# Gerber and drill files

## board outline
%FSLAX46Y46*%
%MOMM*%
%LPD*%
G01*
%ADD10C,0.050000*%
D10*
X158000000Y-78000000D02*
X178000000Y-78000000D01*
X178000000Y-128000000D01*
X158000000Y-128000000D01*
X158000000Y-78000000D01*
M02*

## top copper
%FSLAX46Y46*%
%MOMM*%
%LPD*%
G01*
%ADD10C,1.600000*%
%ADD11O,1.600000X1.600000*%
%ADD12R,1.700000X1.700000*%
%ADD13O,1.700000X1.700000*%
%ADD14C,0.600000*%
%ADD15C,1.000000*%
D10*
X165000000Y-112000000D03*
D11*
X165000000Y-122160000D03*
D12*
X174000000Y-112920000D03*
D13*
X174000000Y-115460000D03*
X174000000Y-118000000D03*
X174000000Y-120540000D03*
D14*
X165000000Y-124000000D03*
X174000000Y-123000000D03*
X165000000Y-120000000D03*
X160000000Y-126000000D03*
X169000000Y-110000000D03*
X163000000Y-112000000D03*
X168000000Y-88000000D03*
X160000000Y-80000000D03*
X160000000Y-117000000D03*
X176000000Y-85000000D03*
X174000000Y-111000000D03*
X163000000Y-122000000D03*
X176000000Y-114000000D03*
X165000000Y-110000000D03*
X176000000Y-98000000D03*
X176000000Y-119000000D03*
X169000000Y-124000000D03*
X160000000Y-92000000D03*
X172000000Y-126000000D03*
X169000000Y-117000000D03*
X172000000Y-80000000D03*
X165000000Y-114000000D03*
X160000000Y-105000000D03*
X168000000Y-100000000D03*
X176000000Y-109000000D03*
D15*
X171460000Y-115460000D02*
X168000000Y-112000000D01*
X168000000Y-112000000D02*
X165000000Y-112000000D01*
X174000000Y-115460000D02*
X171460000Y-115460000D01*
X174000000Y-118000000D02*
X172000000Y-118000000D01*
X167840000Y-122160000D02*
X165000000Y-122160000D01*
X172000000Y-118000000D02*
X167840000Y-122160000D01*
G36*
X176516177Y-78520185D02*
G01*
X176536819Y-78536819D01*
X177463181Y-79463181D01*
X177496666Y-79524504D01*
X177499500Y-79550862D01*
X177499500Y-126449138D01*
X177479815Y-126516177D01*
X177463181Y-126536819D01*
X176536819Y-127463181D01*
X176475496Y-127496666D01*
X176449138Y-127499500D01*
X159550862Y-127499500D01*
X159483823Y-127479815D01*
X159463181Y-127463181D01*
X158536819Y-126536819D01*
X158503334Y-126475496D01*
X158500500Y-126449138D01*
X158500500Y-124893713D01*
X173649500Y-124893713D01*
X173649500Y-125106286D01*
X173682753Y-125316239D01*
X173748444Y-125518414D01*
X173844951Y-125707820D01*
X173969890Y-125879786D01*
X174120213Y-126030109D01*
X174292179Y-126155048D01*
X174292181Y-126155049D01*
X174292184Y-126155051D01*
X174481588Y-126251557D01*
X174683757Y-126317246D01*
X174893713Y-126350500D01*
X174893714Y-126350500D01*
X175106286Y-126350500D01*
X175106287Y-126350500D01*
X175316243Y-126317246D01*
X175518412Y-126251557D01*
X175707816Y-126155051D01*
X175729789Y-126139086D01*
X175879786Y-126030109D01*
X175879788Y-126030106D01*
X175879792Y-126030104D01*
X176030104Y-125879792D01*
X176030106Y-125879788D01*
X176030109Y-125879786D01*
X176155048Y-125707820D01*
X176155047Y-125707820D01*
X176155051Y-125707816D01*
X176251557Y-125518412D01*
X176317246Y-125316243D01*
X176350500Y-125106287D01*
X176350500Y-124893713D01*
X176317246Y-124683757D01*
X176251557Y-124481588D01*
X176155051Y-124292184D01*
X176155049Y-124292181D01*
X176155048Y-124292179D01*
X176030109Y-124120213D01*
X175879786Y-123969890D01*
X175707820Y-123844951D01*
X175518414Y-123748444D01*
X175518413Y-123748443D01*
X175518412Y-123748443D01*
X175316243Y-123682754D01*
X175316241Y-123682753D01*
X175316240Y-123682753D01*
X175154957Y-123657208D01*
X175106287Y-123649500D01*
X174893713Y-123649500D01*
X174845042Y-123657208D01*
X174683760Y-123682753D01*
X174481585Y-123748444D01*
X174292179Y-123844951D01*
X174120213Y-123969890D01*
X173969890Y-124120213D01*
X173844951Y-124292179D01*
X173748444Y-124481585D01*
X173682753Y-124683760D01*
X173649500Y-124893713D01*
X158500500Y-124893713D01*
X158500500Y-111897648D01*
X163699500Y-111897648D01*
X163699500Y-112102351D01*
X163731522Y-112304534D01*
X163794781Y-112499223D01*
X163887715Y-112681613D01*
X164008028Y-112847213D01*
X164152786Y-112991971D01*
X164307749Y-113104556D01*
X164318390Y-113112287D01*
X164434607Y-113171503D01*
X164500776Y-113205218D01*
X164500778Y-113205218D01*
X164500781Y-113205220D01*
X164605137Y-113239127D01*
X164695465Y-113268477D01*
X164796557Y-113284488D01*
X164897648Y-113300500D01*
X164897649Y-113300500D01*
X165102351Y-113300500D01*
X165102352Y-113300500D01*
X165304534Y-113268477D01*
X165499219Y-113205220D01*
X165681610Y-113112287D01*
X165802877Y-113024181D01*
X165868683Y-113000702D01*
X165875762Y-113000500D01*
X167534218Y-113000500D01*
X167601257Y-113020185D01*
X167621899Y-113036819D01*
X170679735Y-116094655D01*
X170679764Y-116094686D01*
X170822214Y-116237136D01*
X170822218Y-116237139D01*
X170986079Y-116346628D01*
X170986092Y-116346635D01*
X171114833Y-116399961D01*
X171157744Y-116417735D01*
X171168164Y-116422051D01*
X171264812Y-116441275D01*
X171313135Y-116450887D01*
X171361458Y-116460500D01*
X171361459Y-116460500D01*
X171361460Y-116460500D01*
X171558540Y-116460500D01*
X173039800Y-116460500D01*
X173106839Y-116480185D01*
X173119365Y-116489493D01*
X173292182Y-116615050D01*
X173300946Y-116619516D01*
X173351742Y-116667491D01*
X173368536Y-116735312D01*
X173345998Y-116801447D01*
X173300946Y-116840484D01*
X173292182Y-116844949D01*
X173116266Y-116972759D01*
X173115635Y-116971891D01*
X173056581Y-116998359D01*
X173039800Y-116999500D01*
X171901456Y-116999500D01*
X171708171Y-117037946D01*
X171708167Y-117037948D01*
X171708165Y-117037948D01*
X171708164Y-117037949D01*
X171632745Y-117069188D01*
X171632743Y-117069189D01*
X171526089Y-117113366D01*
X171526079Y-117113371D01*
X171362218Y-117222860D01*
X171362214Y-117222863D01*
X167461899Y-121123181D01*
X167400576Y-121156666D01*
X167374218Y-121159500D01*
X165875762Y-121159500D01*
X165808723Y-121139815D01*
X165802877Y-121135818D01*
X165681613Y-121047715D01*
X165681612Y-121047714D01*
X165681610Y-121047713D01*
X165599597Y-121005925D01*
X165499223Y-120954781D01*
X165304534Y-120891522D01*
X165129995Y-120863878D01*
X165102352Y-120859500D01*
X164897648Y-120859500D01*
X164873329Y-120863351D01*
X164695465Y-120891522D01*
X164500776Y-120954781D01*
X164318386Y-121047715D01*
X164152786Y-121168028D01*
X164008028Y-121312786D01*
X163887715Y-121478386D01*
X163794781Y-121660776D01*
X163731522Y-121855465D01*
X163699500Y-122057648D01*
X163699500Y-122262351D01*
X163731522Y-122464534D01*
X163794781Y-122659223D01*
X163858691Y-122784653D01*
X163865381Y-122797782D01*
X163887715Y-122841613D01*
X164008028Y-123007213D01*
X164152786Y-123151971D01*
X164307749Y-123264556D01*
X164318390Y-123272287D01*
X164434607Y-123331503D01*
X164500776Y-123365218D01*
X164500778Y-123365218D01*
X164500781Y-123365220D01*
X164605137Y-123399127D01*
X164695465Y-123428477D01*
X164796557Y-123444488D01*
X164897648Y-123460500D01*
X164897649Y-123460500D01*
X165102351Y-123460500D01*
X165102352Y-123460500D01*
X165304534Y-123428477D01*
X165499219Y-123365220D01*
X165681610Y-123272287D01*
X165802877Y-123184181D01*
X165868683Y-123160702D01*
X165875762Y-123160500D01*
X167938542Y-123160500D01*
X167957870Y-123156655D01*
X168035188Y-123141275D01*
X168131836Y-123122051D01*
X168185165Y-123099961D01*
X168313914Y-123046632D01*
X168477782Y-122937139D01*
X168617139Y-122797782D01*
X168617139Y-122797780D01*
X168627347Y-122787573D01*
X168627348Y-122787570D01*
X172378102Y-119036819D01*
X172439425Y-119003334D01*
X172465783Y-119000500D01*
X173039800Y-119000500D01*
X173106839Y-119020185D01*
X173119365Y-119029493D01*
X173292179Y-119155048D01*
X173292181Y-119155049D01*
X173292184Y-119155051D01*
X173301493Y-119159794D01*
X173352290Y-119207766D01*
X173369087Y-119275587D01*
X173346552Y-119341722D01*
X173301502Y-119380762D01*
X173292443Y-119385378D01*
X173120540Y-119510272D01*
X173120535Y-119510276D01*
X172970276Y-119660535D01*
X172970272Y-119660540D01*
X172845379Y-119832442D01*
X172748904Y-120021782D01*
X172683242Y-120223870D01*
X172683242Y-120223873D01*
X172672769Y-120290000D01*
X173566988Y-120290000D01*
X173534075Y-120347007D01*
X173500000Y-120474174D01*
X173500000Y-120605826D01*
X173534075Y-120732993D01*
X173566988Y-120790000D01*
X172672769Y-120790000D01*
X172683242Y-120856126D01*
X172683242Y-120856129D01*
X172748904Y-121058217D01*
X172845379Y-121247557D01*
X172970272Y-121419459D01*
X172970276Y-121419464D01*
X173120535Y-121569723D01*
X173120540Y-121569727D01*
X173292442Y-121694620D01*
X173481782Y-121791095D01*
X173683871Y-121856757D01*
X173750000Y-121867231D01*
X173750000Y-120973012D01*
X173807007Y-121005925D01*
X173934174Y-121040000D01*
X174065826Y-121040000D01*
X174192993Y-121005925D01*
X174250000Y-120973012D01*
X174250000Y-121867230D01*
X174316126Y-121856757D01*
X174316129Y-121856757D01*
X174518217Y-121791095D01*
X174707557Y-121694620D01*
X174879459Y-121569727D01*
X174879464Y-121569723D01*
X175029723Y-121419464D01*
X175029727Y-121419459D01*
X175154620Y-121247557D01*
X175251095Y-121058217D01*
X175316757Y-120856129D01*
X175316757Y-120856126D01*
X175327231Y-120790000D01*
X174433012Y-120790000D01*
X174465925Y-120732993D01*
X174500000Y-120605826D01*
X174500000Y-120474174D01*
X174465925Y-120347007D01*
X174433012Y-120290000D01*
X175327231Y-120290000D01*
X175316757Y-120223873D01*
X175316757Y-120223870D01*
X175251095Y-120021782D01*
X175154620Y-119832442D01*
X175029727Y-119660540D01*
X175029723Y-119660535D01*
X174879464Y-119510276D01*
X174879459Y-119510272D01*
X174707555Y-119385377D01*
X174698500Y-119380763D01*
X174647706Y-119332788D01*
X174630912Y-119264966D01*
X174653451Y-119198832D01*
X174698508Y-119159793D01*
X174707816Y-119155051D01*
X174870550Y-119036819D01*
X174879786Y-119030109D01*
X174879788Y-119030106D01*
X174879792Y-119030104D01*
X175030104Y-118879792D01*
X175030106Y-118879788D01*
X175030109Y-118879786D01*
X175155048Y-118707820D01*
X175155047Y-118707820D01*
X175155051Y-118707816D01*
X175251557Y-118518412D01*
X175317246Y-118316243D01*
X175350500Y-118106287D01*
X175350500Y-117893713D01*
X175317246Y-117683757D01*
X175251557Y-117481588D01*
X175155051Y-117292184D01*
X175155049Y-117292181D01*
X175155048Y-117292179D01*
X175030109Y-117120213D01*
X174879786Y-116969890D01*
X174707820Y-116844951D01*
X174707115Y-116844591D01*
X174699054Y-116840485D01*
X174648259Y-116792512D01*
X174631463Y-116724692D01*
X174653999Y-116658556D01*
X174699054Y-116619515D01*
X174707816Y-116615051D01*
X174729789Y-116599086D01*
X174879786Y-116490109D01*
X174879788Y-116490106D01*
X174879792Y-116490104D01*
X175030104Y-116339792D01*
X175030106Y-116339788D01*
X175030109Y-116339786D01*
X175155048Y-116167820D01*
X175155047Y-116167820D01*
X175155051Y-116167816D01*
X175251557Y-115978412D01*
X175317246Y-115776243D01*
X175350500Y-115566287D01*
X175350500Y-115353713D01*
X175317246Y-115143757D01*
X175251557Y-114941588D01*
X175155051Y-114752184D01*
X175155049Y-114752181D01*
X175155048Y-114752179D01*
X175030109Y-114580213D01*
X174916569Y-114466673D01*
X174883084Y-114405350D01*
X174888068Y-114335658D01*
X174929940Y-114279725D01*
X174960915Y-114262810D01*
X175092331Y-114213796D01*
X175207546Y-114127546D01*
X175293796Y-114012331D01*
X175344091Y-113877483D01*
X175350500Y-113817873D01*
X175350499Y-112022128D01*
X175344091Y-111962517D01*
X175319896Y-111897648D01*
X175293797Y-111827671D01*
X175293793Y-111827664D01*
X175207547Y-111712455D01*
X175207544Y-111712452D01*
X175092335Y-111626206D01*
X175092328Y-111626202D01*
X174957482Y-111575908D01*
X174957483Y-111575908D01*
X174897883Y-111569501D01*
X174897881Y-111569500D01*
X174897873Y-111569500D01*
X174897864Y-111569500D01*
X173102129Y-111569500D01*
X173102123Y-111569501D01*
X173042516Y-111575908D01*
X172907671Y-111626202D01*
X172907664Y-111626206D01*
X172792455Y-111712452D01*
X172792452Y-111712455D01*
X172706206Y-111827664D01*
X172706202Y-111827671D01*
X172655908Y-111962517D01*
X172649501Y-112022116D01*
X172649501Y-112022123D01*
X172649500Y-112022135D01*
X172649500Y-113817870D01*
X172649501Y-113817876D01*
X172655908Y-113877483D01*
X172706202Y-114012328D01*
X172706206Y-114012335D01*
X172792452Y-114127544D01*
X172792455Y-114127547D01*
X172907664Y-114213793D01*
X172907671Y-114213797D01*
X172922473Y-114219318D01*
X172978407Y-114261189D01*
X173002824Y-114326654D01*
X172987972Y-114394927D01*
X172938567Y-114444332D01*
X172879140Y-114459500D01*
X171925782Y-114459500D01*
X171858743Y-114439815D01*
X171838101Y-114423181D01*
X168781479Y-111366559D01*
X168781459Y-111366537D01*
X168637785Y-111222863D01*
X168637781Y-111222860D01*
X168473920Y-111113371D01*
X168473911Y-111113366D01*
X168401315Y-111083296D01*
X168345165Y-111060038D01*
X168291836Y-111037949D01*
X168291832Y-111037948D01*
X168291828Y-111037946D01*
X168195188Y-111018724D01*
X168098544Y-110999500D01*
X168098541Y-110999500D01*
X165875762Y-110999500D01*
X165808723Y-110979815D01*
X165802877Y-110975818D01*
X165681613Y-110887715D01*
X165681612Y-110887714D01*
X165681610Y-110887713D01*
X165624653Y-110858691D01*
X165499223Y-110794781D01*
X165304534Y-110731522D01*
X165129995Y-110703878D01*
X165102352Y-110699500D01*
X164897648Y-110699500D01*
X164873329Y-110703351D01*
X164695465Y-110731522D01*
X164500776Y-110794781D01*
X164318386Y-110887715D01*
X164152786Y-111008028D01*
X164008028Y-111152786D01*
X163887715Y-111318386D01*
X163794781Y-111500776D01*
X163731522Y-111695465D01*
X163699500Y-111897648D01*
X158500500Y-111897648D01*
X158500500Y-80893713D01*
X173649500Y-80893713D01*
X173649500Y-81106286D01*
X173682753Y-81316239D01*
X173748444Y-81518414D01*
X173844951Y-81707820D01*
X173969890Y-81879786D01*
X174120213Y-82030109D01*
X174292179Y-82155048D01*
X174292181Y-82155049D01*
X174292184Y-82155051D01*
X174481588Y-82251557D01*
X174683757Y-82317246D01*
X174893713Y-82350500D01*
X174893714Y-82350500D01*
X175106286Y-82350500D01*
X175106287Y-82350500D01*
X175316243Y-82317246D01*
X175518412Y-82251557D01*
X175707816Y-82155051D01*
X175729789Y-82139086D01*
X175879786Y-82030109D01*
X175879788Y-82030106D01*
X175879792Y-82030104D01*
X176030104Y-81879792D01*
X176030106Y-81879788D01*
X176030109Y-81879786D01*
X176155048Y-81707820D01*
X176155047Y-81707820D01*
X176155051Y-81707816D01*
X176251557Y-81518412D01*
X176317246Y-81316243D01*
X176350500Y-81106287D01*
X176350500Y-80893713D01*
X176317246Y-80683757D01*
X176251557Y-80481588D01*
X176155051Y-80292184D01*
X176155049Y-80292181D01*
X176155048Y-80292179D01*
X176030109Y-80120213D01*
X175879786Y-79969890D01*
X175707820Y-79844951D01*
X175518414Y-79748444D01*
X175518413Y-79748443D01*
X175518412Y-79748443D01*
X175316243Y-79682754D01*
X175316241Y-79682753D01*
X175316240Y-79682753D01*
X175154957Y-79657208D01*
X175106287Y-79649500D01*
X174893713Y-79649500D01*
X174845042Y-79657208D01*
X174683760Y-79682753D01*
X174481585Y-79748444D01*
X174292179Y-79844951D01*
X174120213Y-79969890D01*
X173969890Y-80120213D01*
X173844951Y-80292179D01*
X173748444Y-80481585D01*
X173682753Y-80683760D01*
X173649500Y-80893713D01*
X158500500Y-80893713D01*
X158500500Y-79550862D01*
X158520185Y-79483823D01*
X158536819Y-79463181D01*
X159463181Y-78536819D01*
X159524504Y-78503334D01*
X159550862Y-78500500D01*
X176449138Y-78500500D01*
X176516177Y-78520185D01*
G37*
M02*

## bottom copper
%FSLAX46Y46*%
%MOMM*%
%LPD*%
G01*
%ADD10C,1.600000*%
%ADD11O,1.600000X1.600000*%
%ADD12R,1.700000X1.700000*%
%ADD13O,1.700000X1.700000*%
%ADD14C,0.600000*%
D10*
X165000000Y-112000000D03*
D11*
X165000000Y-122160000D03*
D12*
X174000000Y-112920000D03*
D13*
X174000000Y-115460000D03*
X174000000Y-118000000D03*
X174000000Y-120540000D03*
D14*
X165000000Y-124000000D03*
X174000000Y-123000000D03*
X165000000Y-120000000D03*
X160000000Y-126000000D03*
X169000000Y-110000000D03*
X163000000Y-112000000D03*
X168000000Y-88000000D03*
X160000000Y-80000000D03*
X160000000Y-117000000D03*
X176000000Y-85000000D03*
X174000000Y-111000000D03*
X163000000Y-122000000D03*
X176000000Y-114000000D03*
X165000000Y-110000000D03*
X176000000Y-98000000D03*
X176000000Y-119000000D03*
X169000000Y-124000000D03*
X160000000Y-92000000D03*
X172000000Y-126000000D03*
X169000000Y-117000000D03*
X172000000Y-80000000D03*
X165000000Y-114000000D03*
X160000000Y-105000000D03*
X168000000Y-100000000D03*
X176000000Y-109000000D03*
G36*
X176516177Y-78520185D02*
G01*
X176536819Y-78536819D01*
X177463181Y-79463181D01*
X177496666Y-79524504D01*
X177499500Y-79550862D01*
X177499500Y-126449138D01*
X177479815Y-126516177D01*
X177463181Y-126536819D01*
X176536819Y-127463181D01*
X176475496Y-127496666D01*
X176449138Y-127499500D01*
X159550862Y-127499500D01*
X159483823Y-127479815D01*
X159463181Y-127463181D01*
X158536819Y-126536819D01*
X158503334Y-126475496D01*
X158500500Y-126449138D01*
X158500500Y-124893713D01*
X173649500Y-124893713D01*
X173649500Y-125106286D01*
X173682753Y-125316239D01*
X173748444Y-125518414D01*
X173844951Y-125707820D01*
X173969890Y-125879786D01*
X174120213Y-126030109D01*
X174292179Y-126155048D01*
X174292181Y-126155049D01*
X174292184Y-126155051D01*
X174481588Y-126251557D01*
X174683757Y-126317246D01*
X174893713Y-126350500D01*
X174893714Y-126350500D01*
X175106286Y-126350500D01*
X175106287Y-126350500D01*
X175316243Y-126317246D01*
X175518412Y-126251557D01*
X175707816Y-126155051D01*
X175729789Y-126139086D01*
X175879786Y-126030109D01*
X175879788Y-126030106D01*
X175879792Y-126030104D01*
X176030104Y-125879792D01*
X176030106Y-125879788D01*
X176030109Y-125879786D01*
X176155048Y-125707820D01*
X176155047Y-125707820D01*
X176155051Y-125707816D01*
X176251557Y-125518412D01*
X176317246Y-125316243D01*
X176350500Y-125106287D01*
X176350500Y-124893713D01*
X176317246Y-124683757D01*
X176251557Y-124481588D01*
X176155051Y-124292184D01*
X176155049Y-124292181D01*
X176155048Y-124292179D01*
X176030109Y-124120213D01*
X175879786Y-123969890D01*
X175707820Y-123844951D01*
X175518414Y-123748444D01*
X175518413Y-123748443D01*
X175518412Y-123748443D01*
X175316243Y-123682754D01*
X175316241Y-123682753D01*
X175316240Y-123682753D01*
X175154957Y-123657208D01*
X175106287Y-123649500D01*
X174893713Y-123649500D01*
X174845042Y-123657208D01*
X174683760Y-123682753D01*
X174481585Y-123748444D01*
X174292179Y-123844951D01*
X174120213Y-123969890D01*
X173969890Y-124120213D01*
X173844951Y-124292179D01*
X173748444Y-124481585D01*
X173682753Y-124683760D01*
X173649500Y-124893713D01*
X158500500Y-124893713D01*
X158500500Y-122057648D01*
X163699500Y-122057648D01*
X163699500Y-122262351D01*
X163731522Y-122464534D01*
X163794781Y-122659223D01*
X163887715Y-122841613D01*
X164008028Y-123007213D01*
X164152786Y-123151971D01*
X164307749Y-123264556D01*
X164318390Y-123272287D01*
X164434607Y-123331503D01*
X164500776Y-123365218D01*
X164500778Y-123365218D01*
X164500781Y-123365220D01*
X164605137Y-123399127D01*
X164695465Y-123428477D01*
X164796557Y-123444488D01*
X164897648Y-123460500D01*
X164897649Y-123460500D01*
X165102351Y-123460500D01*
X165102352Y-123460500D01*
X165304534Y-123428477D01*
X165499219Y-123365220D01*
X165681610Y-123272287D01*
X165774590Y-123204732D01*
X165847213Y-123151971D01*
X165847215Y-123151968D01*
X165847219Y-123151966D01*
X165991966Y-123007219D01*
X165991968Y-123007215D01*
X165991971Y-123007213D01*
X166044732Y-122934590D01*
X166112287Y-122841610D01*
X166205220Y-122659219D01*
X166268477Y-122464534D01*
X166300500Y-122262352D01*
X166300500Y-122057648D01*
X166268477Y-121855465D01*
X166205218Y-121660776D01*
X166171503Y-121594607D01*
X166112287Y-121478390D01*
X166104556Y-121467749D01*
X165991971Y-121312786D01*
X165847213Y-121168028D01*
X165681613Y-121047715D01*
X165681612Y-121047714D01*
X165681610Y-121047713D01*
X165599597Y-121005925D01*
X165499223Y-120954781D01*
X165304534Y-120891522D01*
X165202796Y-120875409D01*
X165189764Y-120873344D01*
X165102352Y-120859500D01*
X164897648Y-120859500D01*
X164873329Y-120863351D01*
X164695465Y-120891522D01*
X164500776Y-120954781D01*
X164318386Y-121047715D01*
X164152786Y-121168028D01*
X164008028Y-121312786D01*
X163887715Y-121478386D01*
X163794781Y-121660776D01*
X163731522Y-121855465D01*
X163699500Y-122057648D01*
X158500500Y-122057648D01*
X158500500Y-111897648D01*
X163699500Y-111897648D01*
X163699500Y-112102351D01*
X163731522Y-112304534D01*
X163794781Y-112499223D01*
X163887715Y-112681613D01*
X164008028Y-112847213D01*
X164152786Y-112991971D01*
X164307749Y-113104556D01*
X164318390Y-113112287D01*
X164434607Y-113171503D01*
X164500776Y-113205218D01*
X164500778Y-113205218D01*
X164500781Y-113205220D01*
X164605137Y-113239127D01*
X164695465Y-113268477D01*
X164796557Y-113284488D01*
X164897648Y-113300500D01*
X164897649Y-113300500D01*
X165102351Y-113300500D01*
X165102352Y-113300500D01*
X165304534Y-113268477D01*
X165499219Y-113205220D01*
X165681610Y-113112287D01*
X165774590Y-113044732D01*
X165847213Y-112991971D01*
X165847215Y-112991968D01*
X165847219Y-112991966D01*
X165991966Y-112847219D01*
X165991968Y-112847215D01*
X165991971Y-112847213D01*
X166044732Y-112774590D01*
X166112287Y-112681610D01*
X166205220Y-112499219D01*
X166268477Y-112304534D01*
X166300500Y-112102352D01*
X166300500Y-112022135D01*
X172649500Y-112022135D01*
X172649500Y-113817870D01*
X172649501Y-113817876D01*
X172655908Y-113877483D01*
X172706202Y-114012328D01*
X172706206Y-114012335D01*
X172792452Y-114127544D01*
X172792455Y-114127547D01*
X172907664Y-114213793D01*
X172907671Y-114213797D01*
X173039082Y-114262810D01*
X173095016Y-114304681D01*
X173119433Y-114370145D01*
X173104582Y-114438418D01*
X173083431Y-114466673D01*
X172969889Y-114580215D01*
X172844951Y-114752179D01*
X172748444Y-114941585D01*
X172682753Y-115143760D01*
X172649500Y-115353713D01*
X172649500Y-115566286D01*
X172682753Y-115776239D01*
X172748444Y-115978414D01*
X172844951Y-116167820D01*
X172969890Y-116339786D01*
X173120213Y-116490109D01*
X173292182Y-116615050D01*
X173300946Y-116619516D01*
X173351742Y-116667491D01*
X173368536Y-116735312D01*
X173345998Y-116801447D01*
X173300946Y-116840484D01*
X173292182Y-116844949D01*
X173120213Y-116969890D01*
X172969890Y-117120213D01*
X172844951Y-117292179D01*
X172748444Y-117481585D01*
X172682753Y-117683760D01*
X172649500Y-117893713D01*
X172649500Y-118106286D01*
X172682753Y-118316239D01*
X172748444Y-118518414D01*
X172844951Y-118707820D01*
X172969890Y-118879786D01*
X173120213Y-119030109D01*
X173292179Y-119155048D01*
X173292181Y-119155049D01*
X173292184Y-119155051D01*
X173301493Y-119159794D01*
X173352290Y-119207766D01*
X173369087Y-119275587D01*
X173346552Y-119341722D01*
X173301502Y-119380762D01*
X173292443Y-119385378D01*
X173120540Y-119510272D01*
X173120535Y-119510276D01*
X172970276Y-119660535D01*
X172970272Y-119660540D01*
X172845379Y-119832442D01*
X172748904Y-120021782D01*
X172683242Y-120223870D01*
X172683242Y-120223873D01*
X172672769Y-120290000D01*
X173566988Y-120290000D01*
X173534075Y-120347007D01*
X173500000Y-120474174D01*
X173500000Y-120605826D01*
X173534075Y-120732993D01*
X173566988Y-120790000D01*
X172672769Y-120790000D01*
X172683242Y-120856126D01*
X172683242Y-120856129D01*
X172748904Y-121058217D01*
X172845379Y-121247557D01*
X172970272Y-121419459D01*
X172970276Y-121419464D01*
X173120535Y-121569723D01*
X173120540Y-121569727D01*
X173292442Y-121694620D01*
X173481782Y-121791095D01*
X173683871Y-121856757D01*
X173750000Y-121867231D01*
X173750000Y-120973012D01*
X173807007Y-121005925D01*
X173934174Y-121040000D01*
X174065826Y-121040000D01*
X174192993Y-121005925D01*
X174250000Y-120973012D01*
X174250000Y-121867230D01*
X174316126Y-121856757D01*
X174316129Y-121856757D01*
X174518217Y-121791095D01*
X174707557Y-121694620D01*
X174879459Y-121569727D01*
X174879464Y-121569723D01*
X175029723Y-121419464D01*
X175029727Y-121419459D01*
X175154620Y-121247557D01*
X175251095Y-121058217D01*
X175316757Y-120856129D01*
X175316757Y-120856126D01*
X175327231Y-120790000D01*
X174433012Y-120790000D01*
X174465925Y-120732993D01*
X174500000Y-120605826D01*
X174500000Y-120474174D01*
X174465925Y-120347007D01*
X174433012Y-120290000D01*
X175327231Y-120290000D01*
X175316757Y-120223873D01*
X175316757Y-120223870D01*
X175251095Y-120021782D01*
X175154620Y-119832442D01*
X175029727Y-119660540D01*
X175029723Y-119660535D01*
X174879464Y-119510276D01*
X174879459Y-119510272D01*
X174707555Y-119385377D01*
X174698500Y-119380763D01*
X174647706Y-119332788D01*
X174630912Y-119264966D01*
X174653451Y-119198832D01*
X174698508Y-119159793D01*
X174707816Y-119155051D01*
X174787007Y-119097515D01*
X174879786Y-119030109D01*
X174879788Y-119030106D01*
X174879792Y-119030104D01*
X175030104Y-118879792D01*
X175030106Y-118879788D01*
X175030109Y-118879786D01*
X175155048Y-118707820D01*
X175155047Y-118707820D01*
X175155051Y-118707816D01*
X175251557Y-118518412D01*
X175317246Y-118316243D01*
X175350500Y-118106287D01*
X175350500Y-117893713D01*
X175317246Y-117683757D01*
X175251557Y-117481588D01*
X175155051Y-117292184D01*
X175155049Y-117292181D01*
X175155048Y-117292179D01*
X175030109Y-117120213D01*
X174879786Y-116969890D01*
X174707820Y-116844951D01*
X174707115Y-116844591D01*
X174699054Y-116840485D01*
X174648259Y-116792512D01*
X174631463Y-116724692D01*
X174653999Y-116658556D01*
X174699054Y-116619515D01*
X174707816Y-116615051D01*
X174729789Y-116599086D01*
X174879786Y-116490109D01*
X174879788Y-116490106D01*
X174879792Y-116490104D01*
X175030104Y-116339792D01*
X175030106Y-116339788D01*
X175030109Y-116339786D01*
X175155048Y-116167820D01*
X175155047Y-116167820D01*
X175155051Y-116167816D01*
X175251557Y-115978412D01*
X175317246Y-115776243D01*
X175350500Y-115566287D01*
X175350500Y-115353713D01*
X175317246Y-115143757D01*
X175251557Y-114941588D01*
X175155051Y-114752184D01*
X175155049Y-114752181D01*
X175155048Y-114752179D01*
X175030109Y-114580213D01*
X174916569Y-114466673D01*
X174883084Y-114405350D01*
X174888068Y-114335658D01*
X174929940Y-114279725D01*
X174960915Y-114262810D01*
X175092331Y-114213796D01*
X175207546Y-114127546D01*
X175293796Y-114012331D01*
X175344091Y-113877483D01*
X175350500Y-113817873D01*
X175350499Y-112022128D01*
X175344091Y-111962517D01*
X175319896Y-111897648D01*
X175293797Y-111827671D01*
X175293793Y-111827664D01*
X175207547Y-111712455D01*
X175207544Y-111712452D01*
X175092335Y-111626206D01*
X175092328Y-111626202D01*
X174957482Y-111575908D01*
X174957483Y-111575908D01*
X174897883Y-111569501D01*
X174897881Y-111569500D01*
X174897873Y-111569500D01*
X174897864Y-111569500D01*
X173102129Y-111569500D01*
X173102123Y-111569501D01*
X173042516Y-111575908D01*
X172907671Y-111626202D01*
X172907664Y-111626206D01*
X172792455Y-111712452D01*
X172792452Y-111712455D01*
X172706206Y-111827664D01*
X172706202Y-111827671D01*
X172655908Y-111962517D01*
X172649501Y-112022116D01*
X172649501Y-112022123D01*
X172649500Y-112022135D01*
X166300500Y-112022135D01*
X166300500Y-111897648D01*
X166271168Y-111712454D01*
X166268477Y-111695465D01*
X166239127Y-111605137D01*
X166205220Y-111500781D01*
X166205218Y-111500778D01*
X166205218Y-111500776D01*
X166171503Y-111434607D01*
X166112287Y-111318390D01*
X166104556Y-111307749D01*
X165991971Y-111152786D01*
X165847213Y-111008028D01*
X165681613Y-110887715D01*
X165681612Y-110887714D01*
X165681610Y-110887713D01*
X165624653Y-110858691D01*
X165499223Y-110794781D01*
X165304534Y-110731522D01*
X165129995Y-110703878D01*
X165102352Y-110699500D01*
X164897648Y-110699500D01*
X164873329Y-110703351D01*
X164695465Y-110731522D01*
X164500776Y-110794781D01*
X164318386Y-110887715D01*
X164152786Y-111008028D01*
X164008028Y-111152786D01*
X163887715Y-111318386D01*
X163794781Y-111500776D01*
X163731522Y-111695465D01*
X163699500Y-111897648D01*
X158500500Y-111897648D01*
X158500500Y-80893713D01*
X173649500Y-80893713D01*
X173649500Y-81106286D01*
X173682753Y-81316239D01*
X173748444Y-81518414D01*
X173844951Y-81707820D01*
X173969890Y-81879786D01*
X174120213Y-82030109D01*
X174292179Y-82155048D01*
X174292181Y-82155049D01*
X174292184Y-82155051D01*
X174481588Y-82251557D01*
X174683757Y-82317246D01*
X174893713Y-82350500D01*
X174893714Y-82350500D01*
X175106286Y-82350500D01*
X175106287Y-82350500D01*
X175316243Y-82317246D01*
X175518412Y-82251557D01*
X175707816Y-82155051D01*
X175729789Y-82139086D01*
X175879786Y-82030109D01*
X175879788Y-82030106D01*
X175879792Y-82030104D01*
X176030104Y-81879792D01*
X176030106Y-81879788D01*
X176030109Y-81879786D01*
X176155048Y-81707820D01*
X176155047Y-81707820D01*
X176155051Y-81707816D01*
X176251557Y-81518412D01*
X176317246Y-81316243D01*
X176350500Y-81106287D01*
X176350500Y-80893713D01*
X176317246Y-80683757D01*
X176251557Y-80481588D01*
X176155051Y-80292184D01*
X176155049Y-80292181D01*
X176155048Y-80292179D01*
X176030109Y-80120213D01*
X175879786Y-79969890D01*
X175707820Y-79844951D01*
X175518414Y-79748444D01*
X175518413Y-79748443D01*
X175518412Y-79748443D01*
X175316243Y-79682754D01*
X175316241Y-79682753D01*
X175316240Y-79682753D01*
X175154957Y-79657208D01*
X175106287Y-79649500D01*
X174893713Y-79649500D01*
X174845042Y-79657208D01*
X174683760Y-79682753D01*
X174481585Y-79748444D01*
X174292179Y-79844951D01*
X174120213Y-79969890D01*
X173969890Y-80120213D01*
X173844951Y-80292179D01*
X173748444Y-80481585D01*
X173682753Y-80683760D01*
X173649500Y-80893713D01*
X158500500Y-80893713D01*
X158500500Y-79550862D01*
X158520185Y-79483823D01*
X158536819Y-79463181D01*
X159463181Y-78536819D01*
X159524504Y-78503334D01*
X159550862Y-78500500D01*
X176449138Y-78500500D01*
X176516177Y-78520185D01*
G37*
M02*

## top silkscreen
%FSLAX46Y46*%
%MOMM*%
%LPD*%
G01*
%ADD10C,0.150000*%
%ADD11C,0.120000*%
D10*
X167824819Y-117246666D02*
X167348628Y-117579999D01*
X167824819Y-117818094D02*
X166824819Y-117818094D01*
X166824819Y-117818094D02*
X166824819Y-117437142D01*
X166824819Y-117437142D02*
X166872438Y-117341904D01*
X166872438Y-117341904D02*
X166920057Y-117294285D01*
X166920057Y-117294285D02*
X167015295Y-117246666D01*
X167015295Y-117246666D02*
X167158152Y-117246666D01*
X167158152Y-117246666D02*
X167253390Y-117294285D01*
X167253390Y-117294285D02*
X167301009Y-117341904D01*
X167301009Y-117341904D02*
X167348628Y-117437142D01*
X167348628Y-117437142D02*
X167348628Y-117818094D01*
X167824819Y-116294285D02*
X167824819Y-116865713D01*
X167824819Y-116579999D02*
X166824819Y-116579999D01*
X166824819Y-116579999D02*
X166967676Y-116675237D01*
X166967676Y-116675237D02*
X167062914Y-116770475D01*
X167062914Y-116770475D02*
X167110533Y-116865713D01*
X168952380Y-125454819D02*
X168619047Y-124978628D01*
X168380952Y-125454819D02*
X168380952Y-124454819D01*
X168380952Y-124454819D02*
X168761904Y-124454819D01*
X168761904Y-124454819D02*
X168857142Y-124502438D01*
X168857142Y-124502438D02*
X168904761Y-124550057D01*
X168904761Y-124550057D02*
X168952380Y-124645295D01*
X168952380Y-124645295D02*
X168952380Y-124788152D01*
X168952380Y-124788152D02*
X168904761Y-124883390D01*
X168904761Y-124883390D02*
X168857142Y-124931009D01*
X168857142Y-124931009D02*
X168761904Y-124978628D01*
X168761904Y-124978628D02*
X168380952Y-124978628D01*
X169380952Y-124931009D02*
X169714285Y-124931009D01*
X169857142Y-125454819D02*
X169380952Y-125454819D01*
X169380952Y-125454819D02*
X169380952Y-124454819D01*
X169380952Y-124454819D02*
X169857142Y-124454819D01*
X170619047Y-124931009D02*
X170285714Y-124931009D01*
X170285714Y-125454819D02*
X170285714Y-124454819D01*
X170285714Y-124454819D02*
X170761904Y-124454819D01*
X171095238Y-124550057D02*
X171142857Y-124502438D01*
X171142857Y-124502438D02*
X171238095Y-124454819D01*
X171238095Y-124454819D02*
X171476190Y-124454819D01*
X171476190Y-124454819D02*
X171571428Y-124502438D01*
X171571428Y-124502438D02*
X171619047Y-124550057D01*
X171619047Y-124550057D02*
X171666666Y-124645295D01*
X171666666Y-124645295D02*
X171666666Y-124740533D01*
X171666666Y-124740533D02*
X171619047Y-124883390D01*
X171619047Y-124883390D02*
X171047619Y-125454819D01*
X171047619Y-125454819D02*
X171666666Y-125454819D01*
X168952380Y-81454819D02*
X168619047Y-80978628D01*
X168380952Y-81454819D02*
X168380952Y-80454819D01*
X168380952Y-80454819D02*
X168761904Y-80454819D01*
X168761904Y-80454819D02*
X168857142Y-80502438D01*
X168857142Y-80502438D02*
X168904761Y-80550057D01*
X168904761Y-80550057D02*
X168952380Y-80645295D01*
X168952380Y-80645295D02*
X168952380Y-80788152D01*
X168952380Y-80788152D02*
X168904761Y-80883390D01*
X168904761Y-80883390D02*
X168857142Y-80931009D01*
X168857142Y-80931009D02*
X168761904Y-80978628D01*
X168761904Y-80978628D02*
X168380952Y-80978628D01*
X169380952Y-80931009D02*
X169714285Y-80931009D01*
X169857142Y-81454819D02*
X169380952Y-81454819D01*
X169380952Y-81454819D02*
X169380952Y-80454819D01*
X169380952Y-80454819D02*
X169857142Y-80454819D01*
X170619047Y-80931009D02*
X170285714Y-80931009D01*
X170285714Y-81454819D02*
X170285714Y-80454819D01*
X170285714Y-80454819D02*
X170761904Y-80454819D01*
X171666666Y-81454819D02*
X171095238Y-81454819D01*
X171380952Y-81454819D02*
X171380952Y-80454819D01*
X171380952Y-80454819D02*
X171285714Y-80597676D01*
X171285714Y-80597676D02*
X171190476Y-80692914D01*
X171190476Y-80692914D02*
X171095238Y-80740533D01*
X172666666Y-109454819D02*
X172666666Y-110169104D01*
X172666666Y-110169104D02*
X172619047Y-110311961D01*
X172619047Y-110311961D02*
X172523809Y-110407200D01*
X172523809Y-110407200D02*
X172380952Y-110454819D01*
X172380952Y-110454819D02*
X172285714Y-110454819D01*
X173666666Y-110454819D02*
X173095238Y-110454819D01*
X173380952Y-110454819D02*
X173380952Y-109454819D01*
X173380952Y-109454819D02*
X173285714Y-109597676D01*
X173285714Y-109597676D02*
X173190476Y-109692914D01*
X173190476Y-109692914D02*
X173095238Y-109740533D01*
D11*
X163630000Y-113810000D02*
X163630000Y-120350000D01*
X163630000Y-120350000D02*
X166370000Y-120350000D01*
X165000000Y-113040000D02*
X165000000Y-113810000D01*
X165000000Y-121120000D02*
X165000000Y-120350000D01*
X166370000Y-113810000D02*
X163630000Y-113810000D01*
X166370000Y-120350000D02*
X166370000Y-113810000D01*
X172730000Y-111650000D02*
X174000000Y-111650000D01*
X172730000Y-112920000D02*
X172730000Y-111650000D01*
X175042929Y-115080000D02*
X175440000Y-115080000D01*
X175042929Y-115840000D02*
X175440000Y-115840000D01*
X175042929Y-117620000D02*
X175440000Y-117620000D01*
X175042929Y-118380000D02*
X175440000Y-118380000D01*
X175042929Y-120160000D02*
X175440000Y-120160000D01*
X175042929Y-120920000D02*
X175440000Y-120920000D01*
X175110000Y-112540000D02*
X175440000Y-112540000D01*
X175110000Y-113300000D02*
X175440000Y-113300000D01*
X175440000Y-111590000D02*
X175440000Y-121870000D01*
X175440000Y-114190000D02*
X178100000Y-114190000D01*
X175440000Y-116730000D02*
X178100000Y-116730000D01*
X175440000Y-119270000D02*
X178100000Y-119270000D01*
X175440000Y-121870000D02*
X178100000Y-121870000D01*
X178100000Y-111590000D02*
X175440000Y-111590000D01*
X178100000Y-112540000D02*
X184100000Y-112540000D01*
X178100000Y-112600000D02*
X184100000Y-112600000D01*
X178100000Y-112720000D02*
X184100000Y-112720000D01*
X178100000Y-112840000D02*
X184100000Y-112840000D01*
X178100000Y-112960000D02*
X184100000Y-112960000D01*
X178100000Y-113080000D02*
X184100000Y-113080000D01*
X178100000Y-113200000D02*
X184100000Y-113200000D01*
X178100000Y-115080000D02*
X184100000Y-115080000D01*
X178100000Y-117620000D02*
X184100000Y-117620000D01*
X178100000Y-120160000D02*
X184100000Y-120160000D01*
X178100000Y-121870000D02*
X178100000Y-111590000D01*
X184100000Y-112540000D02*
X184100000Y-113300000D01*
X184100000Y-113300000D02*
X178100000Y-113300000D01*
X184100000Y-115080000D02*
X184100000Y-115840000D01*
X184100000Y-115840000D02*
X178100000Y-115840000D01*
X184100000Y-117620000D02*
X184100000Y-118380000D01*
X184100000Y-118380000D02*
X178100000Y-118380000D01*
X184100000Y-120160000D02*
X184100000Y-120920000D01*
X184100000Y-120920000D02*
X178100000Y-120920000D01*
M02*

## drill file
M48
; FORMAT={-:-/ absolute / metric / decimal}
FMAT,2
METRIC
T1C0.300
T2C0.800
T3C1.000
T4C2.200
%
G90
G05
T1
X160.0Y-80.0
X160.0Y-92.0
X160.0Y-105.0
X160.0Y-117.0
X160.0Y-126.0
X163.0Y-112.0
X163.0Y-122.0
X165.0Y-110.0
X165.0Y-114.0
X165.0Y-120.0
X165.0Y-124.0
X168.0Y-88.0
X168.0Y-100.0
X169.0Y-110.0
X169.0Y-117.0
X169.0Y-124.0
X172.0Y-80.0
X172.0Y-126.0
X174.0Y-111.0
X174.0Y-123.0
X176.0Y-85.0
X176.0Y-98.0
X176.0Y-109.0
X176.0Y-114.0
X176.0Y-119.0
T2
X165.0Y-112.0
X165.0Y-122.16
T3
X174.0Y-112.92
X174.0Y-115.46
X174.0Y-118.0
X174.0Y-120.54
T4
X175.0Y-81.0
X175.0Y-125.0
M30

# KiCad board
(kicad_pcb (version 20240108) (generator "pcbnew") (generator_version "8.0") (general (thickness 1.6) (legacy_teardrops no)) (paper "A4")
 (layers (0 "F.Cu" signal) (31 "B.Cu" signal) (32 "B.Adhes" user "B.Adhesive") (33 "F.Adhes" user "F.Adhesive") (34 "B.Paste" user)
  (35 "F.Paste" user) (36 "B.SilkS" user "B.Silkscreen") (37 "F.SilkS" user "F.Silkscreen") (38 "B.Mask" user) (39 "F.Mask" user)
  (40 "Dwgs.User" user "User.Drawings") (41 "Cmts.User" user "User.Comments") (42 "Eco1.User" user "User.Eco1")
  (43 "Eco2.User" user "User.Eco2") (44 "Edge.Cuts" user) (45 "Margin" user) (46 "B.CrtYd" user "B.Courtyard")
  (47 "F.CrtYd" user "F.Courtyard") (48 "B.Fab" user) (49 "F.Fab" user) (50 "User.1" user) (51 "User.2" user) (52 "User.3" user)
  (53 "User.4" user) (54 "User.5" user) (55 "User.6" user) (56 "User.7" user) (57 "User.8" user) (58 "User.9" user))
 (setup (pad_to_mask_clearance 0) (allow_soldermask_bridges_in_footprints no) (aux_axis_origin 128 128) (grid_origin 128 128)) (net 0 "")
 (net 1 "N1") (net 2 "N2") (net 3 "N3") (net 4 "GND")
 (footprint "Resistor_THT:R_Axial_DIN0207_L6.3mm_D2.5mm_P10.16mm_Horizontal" (layer "F.Cu") (at 165 112 -90)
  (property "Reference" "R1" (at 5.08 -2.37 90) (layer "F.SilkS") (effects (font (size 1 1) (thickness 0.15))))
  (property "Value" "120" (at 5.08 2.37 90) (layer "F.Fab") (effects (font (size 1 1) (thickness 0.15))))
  (fp_line (start 1.81 1.37) (end 8.35 1.37) (stroke (width 0.12) (type solid)) (layer "F.SilkS"))
  (fp_line (start 8.35 1.37) (end 8.35 -1.37) (stroke (width 0.12) (type solid)) (layer "F.SilkS"))
  (fp_line (start 1.04 0) (end 1.81 0) (stroke (width 0.12) (type solid)) (layer "F.SilkS"))
  (fp_line (start 9.12 0) (end 8.35 0) (stroke (width 0.12) (type solid)) (layer "F.SilkS"))
  (fp_line (start 1.81 -1.37) (end 1.81 1.37) (stroke (width 0.12) (type solid)) (layer "F.SilkS"))
  (fp_line (start 8.35 -1.37) (end 1.81 -1.37) (stroke (width 0.12) (type solid)) (layer "F.SilkS"))
  (pad "1" thru_hole circle (at 0 0 270) (size 1.6 1.6) (drill 0.8) (layers "*.Cu" "*.Mask") (remove_unused_layers no) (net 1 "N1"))
  (pad "2" thru_hole oval (at 10.16 0 270) (size 1.6 1.6) (drill 0.8) (layers "*.Cu" "*.Mask") (remove_unused_layers no) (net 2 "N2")))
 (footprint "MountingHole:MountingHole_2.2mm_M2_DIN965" (layer "F.Cu") (at 175 125)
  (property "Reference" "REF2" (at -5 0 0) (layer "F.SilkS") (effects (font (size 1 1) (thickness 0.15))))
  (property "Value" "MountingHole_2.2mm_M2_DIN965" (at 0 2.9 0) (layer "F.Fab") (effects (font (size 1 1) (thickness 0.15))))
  (pad "" np_thru_hole circle (at 0 0) (size 2.2 2.2) (drill 2.2) (layers "*.Cu" "*.Mask")))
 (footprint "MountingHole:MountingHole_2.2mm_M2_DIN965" (layer "F.Cu") (at 175 81)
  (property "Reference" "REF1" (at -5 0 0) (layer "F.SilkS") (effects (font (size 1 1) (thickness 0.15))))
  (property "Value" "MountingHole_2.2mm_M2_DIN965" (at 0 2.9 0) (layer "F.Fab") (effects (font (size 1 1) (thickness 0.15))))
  (pad "" np_thru_hole circle (at 0 0) (size 2.2 2.2) (drill 2.2) (layers "*.Cu" "*.Mask")))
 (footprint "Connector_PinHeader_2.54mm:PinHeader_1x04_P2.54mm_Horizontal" (layer "F.Cu") (at 174 112.92)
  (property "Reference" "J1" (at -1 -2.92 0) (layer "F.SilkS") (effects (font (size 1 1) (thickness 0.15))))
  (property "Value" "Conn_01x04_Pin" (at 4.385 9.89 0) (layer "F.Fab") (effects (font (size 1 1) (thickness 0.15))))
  (fp_line (start -1.27 -1.27) (end 0 -1.27) (stroke (width 0.12) (type solid)) (layer "F.SilkS"))
  (fp_line (start -1.27 0) (end -1.27 -1.27) (stroke (width 0.12) (type solid)) (layer "F.SilkS"))
  (fp_line (start 1.042929 2.16) (end 1.44 2.16) (stroke (width 0.12) (type solid)) (layer "F.SilkS"))
  (fp_line (start 1.042929 2.92) (end 1.44 2.92) (stroke (width 0.12) (type solid)) (layer "F.SilkS"))
  (fp_line (start 1.042929 4.7) (end 1.44 4.7) (stroke (width 0.12) (type solid)) (layer "F.SilkS"))
  (fp_line (start 1.042929 5.46) (end 1.44 5.46) (stroke (width 0.12) (type solid)) (layer "F.SilkS"))
  (fp_line (start 1.042929 7.24) (end 1.44 7.24) (stroke (width 0.12) (type solid)) (layer "F.SilkS"))
  (fp_line (start 1.042929 8) (end 1.44 8) (stroke (width 0.12) (type solid)) (layer "F.SilkS"))
  (fp_line (start 1.11 -0.38) (end 1.44 -0.38) (stroke (width 0.12) (type solid)) (layer "F.SilkS"))
  (fp_line (start 1.11 0.38) (end 1.44 0.38) (stroke (width 0.12) (type solid)) (layer "F.SilkS"))
  (fp_line (start 1.44 -1.33) (end 1.44 8.95) (stroke (width 0.12) (type solid)) (layer "F.SilkS"))
  (fp_line (start 1.44 1.27) (end 4.1 1.27) (stroke (width 0.12) (type solid)) (layer "F.SilkS"))
  (fp_line (start 1.44 3.81) (end 4.1 3.81) (stroke (width 0.12) (type solid)) (layer "F.SilkS"))
  (fp_line (start 1.44 6.35) (end 4.1 6.35) (stroke (width 0.12) (type solid)) (layer "F.SilkS"))
  (fp_line (start 1.44 8.95) (end 4.1 8.95) (stroke (width 0.12) (type solid)) (layer "F.SilkS"))
  (fp_line (start 4.1 -1.33) (end 1.44 -1.33) (stroke (width 0.12) (type solid)) (layer "F.SilkS"))
  (fp_line (start 4.1 -0.38) (end 10.1 -0.38) (stroke (width 0.12) (type solid)) (layer "F.SilkS"))
  (fp_line (start 4.1 -0.32) (end 10.1 -0.32) (stroke (width 0.12) (type solid)) (layer "F.SilkS"))
  (fp_line (start 4.1 -0.2) (end 10.1 -0.2) (stroke (width 0.12) (type solid)) (layer "F.SilkS"))
  (fp_line (start 4.1 -0.08) (end 10.1 -0.08) (stroke (width 0.12) (type solid)) (layer "F.SilkS"))
  (fp_line (start 4.1 0.04) (end 10.1 0.04) (stroke (width 0.12) (type solid)) (layer "F.SilkS"))
  (fp_line (start 4.1 0.16) (end 10.1 0.16) (stroke (width 0.12) (type solid)) (layer "F.SilkS"))
  (fp_line (start 4.1 0.28) (end 10.1 0.28) (stroke (width 0.12) (type solid)) (layer "F.SilkS"))
  (fp_line (start 4.1 2.16) (end 10.1 2.16) (stroke (width 0.12) (type solid)) (layer "F.SilkS"))
  (fp_line (start 4.1 4.7) (end 10.1 4.7) (stroke (width 0.12) (type solid)) (layer "F.SilkS"))
  (fp_line (start 4.1 7.24) (end 10.1 7.24) (stroke (width 0.12) (type solid)) (layer "F.SilkS"))
  (fp_line (start 4.1 8.95) (end 4.1 -1.33) (stroke (width 0.12) (type solid)) (layer "F.SilkS"))
  (fp_line (start 10.1 -0.38) (end 10.1 0.38) (stroke (width 0.12) (type solid)) (layer "F.SilkS"))
  (fp_line (start 10.1 0.38) (end 4.1 0.38) (stroke (width 0.12) (type solid)) (layer "F.SilkS"))
  (fp_line (start 10.1 2.16) (end 10.1 2.92) (stroke (width 0.12) (type solid)) (layer "F.SilkS"))
  (fp_line (start 10.1 2.92) (end 4.1 2.92) (stroke (width 0.12) (type solid)) (layer "F.SilkS"))
  (fp_line (start 10.1 4.7) (end 10.1 5.46) (stroke (width 0.12) (type solid)) (layer "F.SilkS"))
  (fp_line (start 10.1 5.46) (end 4.1 5.46) (stroke (width 0.12) (type solid)) (layer "F.SilkS"))
  (fp_line (start 10.1 7.24) (end 10.1 8) (stroke (width 0.12) (type solid)) (layer "F.SilkS"))
  (fp_line (start 10.1 8) (end 4.1 8) (stroke (width 0.12) (type solid)) (layer "F.SilkS"))
  (pad "1" thru_hole rect (at 0 0) (size 1.7 1.7) (drill 1) (layers "*.Cu" "*.Mask") (remove_unused_layers no) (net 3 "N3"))
  (pad "2" thru_hole oval (at 0 2.54) (size 1.7 1.7) (drill 1) (layers "*.Cu" "*.Mask") (remove_unused_layers no) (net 1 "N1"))
  (pad "3" thru_hole oval (at 0 5.08) (size 1.7 1.7) (drill 1) (layers "*.Cu" "*.Mask") (remove_unused_layers no) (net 2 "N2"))
  (pad "4" thru_hole oval (at 0 7.62) (size 1.7 1.7) (drill 1) (layers "*.Cu" "*.Mask") (remove_unused_layers no) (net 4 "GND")))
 (gr_rect (start 158 78) (end 178 128) (stroke (width 0.05) (type default)) (fill none) (layer "Edge.Cuts"))
 (segment (start 171.46 115.46) (end 168 112) (width 1) (layer "F.Cu") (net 1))
 (segment (start 168 112) (end 165 112) (width 1) (layer "F.Cu") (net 1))
 (segment (start 174 115.46) (end 171.46 115.46) (width 1) (layer "F.Cu") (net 1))
 (segment (start 174 118) (end 172 118) (width 1) (layer "F.Cu") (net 2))
 (segment (start 167.84 122.16) (end 165 122.16) (width 1) (layer "F.Cu") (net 2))
 (segment (start 172 118) (end 167.84 122.16) (width 1) (layer "F.Cu") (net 2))
 (via (at 165 124) (size 0.6) (drill 0.3) (layers "F.Cu" "B.Cu") (free yes) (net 4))
 (via (at 174 123) (size 0.6) (drill 0.3) (layers "F.Cu" "B.Cu") (free yes) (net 4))
 (via (at 165 120) (size 0.6) (drill 0.3) (layers "F.Cu" "B.Cu") (free yes) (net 4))
 (via (at 160 126) (size 0.6) (drill 0.3) (layers "F.Cu" "B.Cu") (free yes) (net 4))
 (via (at 169 110) (size 0.6) (drill 0.3) (layers "F.Cu" "B.Cu") (free yes) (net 4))
 (via (at 163 112) (size 0.6) (drill 0.3) (layers "F.Cu" "B.Cu") (free yes) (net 4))
 (via (at 168 88) (size 0.6) (drill 0.3) (layers "F.Cu" "B.Cu") (free yes) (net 4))
 (via (at 160 80) (size 0.6) (drill 0.3) (layers "F.Cu" "B.Cu") (free yes) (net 4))
 (via (at 160 117) (size 0.6) (drill 0.3) (layers "F.Cu" "B.Cu") (free yes) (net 4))
 (via (at 176 85) (size 0.6) (drill 0.3) (layers "F.Cu" "B.Cu") (free yes) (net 4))
 (via (at 174 111) (size 0.6) (drill 0.3) (layers "F.Cu" "B.Cu") (free yes) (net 4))
 (via (at 163 122) (size 0.6) (drill 0.3) (layers "F.Cu" "B.Cu") (free yes) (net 4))
 (via (at 176 114) (size 0.6) (drill 0.3) (layers "F.Cu" "B.Cu") (free yes) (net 4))
 (via (at 165 110) (size 0.6) (drill 0.3) (layers "F.Cu" "B.Cu") (free yes) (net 4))
 (via (at 176 98) (size 0.6) (drill 0.3) (layers "F.Cu" "B.Cu") (free yes) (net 4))
 (via (at 176 119) (size 0.6) (drill 0.3) (layers "F.Cu" "B.Cu") (free yes) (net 4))
 (via (at 169 124) (size 0.6) (drill 0.3) (layers "F.Cu" "B.Cu") (free yes) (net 4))
 (via (at 160 92) (size 0.6) (drill 0.3) (layers "F.Cu" "B.Cu") (free yes) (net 4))
 (via (at 172 126) (size 0.6) (drill 0.3) (layers "F.Cu" "B.Cu") (free yes) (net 4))
 (via (at 169 117) (size 0.6) (drill 0.3) (layers "F.Cu" "B.Cu") (free yes) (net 4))
 (via (at 172 80) (size 0.6) (drill 0.3) (layers "F.Cu" "B.Cu") (free yes) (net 4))
 (via (at 165 114) (size 0.6) (drill 0.3) (layers "F.Cu" "B.Cu") (free yes) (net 4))
 (via (at 160 105) (size 0.6) (drill 0.3) (layers "F.Cu" "B.Cu") (free yes) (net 4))
 (via (at 168 100) (size 0.6) (drill 0.3) (layers "F.Cu" "B.Cu") (free yes) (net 4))
 (via (at 176 109) (size 0.6) (drill 0.3) (layers "F.Cu" "B.Cu") (free yes) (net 4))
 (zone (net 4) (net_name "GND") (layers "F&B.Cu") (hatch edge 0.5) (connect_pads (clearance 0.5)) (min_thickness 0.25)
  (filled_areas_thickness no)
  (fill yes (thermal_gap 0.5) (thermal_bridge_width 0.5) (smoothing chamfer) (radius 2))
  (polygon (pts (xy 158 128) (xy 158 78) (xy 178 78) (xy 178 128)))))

